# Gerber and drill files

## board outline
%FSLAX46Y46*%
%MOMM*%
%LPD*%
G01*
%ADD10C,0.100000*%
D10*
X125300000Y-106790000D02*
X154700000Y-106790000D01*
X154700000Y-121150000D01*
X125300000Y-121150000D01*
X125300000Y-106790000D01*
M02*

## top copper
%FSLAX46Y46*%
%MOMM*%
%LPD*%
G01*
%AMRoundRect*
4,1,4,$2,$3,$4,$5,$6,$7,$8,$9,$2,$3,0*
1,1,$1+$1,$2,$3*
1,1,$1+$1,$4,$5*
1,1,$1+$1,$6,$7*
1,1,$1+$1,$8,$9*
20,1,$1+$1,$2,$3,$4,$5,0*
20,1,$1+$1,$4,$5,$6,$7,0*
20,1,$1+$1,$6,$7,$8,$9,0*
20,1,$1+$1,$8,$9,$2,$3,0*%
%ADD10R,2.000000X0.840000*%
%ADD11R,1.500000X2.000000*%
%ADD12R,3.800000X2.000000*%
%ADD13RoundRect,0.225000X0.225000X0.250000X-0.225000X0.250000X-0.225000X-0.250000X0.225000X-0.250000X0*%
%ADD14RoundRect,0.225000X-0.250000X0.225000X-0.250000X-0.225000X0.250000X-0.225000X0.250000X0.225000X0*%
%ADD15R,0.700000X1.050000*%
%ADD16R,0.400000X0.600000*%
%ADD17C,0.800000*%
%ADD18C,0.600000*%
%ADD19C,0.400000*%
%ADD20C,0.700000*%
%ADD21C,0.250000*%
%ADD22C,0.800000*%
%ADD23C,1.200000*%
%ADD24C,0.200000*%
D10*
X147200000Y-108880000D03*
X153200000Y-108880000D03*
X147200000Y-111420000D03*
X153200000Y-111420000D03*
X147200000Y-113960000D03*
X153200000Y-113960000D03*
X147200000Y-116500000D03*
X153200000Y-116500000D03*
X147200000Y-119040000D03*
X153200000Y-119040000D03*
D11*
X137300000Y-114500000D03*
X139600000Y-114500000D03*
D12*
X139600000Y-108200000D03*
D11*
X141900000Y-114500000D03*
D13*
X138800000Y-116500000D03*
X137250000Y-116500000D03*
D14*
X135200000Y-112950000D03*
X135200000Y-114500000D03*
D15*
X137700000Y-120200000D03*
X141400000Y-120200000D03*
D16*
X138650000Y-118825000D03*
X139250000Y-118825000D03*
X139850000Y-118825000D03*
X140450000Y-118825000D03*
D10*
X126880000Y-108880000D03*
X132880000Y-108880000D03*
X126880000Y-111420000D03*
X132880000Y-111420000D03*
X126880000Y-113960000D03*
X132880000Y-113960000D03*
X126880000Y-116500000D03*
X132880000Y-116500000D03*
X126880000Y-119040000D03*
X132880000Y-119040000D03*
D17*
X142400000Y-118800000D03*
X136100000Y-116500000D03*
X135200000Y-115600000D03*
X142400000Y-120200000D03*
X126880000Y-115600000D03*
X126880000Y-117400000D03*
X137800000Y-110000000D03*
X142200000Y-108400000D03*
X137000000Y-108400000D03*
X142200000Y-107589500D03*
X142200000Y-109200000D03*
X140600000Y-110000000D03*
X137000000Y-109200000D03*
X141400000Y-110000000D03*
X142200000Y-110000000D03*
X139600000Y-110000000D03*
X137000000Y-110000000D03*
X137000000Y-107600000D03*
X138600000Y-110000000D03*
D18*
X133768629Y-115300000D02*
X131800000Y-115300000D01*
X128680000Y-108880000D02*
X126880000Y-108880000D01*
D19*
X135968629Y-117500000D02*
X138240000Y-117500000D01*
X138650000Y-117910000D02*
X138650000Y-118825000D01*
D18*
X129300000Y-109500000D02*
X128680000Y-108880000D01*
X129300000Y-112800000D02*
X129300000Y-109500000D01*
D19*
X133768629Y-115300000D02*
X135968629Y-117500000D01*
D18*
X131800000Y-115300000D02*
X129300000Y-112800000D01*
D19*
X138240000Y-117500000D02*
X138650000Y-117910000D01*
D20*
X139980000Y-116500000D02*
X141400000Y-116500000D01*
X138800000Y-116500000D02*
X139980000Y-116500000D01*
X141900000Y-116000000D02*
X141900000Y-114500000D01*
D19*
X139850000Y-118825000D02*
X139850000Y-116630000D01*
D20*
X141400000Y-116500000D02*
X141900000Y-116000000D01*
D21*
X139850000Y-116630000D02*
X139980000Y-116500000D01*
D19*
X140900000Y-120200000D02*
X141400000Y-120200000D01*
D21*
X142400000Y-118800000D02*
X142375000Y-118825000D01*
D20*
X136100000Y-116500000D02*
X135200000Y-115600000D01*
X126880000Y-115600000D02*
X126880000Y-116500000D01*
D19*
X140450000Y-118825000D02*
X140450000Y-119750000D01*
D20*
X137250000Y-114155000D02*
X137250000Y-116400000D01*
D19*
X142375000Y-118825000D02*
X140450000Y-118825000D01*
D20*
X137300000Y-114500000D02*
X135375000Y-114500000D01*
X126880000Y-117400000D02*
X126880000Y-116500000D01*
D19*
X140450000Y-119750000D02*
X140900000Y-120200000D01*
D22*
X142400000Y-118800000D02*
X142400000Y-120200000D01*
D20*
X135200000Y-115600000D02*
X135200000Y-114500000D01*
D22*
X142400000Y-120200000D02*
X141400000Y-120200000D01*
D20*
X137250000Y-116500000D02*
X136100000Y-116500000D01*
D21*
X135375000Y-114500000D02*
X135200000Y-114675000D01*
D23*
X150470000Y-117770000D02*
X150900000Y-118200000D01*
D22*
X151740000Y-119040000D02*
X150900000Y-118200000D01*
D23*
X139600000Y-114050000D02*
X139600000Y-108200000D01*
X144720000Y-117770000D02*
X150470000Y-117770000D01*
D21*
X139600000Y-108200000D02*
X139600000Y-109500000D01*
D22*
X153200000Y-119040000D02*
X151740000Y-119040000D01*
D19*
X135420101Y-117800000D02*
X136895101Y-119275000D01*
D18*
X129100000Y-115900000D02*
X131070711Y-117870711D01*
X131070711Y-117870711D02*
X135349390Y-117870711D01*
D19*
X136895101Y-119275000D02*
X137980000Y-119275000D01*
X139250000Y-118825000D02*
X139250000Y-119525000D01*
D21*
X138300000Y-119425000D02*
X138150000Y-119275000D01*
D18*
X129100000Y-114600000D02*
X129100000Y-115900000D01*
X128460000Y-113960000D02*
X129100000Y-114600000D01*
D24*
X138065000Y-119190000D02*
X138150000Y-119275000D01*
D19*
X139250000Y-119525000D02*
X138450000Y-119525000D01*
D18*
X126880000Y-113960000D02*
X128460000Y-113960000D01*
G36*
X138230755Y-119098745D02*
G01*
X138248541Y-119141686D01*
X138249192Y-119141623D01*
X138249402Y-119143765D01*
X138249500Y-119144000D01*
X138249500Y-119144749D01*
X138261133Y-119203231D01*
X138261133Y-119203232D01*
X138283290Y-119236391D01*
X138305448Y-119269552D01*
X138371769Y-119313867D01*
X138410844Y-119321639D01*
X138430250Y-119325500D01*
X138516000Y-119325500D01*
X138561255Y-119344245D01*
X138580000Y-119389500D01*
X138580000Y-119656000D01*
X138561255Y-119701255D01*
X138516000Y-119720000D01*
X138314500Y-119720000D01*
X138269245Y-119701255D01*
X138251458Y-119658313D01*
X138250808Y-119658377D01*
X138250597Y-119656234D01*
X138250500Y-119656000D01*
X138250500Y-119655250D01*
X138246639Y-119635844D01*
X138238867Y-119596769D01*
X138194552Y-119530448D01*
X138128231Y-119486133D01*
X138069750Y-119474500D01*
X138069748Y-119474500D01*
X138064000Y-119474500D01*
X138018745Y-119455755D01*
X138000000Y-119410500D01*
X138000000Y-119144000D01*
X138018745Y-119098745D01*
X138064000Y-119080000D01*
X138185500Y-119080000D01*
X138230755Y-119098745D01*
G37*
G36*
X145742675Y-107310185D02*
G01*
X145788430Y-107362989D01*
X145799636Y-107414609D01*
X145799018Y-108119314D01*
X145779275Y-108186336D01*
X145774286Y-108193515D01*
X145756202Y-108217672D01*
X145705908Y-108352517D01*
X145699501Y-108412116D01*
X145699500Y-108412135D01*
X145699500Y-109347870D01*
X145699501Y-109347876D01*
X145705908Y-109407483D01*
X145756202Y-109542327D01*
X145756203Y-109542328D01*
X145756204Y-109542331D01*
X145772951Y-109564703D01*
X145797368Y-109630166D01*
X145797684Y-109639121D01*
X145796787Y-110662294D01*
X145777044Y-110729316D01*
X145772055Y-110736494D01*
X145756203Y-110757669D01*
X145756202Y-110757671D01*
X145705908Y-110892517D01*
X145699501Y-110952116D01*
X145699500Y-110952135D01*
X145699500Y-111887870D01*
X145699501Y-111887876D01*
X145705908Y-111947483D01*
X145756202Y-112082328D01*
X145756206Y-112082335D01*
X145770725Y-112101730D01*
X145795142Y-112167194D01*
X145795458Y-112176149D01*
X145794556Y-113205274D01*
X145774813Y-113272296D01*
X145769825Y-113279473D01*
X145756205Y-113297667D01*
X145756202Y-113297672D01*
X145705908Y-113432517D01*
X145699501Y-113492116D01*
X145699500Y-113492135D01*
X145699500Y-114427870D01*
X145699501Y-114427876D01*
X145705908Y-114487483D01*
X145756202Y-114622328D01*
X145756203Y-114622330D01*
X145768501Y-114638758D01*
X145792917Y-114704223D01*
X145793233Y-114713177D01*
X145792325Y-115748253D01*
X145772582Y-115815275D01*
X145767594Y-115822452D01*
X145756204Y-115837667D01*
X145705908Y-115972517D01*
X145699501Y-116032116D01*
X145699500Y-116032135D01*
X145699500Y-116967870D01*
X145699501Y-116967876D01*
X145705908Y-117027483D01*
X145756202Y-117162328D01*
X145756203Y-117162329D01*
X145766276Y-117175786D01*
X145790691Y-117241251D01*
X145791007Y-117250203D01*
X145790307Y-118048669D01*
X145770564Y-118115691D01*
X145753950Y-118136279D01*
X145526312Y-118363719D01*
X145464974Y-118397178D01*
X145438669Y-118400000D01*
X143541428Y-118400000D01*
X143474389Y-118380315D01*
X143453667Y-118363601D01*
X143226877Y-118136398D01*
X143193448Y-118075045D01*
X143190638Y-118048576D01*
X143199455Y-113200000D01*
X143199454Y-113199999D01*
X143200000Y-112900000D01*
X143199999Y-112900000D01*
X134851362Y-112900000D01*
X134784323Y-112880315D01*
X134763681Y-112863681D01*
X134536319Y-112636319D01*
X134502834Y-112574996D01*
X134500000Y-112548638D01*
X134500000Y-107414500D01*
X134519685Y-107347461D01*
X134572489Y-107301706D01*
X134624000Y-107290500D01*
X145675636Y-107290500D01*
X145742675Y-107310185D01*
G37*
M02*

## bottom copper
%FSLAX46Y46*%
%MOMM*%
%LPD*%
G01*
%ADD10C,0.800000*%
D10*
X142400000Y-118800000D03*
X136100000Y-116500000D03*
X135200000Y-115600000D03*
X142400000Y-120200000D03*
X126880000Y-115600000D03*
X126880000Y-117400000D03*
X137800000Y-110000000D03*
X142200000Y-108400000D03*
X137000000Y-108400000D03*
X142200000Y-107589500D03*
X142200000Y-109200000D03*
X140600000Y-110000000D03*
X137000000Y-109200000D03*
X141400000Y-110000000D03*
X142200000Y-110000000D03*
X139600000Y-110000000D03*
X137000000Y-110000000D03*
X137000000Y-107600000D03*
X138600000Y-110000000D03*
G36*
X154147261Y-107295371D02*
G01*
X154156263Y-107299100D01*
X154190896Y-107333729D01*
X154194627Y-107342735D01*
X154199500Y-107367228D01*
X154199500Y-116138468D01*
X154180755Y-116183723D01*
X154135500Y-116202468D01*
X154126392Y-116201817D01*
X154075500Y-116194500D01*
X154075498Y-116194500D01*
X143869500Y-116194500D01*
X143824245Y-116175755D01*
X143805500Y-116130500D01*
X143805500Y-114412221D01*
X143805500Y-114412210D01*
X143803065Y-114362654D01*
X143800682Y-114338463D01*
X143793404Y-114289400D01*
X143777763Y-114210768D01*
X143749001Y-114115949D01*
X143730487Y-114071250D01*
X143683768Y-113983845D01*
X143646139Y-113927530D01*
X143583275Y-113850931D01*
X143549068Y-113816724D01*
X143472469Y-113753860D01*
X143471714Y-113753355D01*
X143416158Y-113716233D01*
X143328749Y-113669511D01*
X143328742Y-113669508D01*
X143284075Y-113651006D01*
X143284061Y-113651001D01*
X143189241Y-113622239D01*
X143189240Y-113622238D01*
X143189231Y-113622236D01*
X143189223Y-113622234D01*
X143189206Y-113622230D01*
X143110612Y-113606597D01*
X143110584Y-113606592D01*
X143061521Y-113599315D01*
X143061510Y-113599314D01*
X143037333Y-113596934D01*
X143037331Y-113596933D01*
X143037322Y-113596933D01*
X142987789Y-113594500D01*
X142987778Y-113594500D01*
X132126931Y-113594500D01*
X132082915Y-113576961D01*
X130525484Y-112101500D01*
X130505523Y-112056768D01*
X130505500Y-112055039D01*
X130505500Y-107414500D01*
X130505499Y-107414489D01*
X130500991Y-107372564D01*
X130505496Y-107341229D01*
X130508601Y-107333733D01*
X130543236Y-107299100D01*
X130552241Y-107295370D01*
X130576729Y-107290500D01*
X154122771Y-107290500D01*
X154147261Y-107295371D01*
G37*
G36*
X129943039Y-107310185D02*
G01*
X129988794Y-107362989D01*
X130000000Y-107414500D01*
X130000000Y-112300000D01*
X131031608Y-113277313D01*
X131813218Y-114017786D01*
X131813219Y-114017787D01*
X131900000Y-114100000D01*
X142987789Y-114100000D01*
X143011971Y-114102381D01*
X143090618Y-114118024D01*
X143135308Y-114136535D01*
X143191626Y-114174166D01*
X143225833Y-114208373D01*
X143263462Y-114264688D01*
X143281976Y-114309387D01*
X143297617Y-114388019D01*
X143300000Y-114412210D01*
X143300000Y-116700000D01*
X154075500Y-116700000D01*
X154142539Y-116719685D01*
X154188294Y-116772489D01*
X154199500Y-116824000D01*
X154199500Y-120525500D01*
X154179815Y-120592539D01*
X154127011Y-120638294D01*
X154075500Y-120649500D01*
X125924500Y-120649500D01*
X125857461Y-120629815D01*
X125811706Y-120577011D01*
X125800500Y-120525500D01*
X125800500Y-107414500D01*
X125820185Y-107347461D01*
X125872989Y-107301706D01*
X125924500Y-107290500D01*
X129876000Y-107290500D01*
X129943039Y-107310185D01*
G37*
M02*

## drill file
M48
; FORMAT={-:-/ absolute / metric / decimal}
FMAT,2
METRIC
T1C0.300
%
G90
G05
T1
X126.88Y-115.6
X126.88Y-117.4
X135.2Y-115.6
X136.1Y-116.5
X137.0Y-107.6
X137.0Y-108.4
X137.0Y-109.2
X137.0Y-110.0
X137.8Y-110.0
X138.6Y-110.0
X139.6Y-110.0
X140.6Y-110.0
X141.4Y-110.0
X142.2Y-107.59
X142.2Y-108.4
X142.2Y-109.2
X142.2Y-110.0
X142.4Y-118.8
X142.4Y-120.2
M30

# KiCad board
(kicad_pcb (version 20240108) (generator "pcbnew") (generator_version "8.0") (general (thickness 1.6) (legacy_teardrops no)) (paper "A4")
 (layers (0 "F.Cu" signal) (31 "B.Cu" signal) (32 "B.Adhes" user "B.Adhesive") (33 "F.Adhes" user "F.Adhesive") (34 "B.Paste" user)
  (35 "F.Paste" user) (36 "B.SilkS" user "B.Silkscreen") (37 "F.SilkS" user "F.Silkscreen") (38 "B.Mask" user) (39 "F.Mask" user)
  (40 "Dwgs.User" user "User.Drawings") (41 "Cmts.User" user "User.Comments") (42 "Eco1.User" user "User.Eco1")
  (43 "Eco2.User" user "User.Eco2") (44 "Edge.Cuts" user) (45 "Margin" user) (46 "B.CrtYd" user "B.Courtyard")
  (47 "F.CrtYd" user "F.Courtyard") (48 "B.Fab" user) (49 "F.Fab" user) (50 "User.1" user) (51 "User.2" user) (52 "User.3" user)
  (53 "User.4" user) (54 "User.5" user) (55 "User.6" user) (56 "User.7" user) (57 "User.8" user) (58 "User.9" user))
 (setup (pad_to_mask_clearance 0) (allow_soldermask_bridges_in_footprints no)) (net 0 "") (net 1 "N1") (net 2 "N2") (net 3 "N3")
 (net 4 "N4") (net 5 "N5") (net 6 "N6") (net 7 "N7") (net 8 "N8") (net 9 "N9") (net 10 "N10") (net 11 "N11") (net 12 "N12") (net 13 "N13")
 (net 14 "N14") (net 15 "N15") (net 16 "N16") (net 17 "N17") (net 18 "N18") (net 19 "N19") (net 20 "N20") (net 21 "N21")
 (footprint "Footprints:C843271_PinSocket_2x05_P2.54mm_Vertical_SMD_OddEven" (layer "F.Cu") (at 150.2 113.96)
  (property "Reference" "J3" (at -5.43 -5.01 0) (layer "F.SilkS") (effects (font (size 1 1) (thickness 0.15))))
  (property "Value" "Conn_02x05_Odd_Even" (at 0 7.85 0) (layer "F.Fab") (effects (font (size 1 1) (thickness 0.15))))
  (pad "1" smd rect (at -3 -5.08) (size 2 0.84) (layers "F.Cu" "F.Paste" "F.Mask") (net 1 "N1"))
  (pad "2" smd rect (at 3 -5.08) (size 2 0.84) (layers "F.Cu" "F.Paste" "F.Mask") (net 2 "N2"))
  (pad "3" smd rect (at -3 -2.54) (size 2 0.84) (layers "F.Cu" "F.Paste" "F.Mask") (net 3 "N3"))
  (pad "4" smd rect (at 3 -2.54) (size 2 0.84) (layers "F.Cu" "F.Paste" "F.Mask") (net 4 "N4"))
  (pad "5" smd rect (at -3 0) (size 2 0.84) (layers "F.Cu" "F.Paste" "F.Mask") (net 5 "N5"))
  (pad "6" smd rect (at 3 0) (size 2 0.84) (layers "F.Cu" "F.Paste" "F.Mask") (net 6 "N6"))
  (pad "7" smd rect (at -3 2.54) (size 2 0.84) (layers "F.Cu" "F.Paste" "F.Mask") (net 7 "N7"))
  (pad "8" smd rect (at 3 2.54) (size 2 0.84) (layers "F.Cu" "F.Paste" "F.Mask") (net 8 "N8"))
  (pad "9" smd rect (at -3 5.08) (size 2 0.84) (layers "F.Cu" "F.Paste" "F.Mask") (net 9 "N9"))
  (pad "10" smd rect (at 3 5.08) (size 2 0.84) (layers "F.Cu" "F.Paste" "F.Mask") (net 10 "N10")))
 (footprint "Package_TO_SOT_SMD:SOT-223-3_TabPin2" (layer "F.Cu") (at 139.6 111.35 90)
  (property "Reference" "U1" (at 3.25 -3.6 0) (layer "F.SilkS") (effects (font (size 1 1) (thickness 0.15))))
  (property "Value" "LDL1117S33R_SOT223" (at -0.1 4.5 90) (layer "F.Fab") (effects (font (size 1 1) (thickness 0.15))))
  (pad "1" smd rect (at -3.15 -2.3 90) (size 2 1.5) (layers "F.Cu" "F.Paste" "F.Mask") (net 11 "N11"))
  (pad "2" smd rect (at -3.15 0 90) (size 2 1.5) (layers "F.Cu" "F.Paste" "F.Mask") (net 10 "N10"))
  (pad "2" smd rect (at 3.15 0 90) (size 2 3.8) (layers "F.Cu" "F.Paste" "F.Mask") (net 10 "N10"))
  (pad "3" smd rect (at -3.15 2.3 90) (size 2 1.5) (layers "F.Cu" "F.Paste" "F.Mask") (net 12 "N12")))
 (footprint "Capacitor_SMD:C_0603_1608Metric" (layer "F.Cu") (at 138.025 116.5 180)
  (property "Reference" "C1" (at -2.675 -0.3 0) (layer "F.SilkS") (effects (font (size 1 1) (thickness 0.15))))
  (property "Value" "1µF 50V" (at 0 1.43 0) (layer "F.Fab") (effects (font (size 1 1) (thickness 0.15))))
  (pad "1" smd roundrect (at -0.775 0 180) (size 0.9 0.95) (layers "F.Cu" "F.Paste" "F.Mask") (roundrect_rratio 0.25) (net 12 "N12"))
  (pad "2" smd roundrect (at 0.775 0 180) (size 0.9 0.95) (layers "F.Cu" "F.Paste" "F.Mask") (roundrect_rratio 0.25) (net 11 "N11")))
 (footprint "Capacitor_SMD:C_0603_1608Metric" (layer "F.Cu") (at 135.2 113.725 -90)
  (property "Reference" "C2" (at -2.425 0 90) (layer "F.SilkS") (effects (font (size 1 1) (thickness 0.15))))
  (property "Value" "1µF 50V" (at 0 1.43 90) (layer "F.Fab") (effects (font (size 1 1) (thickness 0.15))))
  (pad "1" smd roundrect (at -0.775 0 270) (size 0.9 0.95) (layers "F.Cu" "F.Paste" "F.Mask") (roundrect_rratio 0.25) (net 10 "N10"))
  (pad "2" smd roundrect (at 0.775 0 270) (size 0.9 0.95) (layers "F.Cu" "F.Paste" "F.Mask") (roundrect_rratio 0.25) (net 11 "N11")))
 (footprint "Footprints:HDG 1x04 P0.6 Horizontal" (layer "F.Cu") (at 139.55 120.575)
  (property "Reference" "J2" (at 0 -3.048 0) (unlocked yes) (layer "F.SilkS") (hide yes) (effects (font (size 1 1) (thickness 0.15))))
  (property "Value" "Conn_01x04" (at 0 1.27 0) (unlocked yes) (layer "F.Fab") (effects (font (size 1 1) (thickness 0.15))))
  (pad "" smd rect (at -1.85 -0.375 90) (size 1.05 0.7) (layers "F.Cu" "F.Paste" "F.Mask") (thermal_bridge_angle 45))
  (pad "" smd rect (at 1.85 -0.375 90) (size 1.05 0.7) (layers "F.Cu" "F.Paste" "F.Mask") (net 11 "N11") (thermal_bridge_angle 45))
  (pad "1" smd rect (at -0.9 -1.75 90) (size 0.6 0.4) (layers "F.Cu" "F.Paste" "F.Mask") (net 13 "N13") (thermal_bridge_angle 45))
  (pad "2" smd rect (at -0.3 -1.75 90) (size 0.6 0.4) (layers "F.Cu" "F.Paste" "F.Mask") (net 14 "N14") (thermal_bridge_angle 45))
  (pad "3" smd rect (at 0.3 -1.75 90) (size 0.6 0.4) (layers "F.Cu" "F.Paste" "F.Mask") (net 12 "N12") (thermal_bridge_angle 45))
  (pad "4" smd rect (at 0.9 -1.75 90) (size 0.6 0.4) (layers "F.Cu" "F.Paste" "F.Mask") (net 11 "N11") (thermal_bridge_angle 45)))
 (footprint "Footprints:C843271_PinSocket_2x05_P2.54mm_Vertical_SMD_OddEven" (layer "F.Cu") (at 129.88 113.96)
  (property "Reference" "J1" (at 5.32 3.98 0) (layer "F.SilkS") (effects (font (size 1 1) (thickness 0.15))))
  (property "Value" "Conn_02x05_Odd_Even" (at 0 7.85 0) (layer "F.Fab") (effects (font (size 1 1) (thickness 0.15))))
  (pad "1" smd rect (at -3 -5.08) (size 2 0.84) (layers "F.Cu" "F.Paste" "F.Mask") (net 13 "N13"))
  (pad "2" smd rect (at 3 -5.08) (size 2 0.84) (layers "F.Cu" "F.Paste" "F.Mask") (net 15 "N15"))
  (pad "3" smd rect (at -3 -2.54) (size 2 0.84) (layers "F.Cu" "F.Paste" "F.Mask") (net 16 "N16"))
  (pad "4" smd rect (at 3 -2.54) (size 2 0.84) (layers "F.Cu" "F.Paste" "F.Mask") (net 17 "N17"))
  (pad "5" smd rect (at -3 0) (size 2 0.84) (layers "F.Cu" "F.Paste" "F.Mask") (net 14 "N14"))
  (pad "6" smd rect (at 3 0) (size 2 0.84) (layers "F.Cu" "F.Paste" "F.Mask") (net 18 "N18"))
  (pad "7" smd rect (at -3 2.54) (size 2 0.84) (layers "F.Cu" "F.Paste" "F.Mask") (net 11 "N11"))
  (pad "8" smd rect (at 3 2.54) (size 2 0.84) (layers "F.Cu" "F.Paste" "F.Mask") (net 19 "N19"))
  (pad "9" smd rect (at -3 5.08) (size 2 0.84) (layers "F.Cu" "F.Paste" "F.Mask") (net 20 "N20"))
  (pad "10" smd rect (at 3 5.08) (size 2 0.84) (layers "F.Cu" "F.Paste" "F.Mask") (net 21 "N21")))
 (gr_rect (start 125.3 106.79) (end 154.7 121.15) (stroke (width 0.1) (type default)) (fill none) (layer "Edge.Cuts"))
 (segment (start 133.768629 115.3) (end 131.8 115.3) (width 0.6) (layer "F.Cu") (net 13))
 (segment (start 128.68 108.88) (end 126.88 108.88) (width 0.6) (layer "F.Cu") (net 13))
 (segment (start 135.968629 117.5) (end 138.24 117.5) (width 0.4) (layer "F.Cu") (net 13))
 (segment (start 138.65 117.91) (end 138.65 118.825) (width 0.4) (layer "F.Cu") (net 13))
 (segment (start 129.3 109.5) (end 128.68 108.88) (width 0.6) (layer "F.Cu") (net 13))
 (segment (start 129.3 112.8) (end 129.3 109.5) (width 0.6) (layer "F.Cu") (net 13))
 (segment (start 133.768629 115.3) (end 135.968629 117.5) (width 0.4) (layer "F.Cu") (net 13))
 (segment (start 131.8 115.3) (end 129.3 112.8) (width 0.6) (layer "F.Cu") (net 13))
 (segment (start 138.24 117.5) (end 138.65 117.91) (width 0.4) (layer "F.Cu") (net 13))
 (segment (start 139.98 116.5) (end 141.4 116.5) (width 0.7) (layer "F.Cu") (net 12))
 (segment (start 138.8 116.5) (end 139.98 116.5) (width 0.7) (layer "F.Cu") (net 12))
 (segment (start 141.9 116) (end 141.9 114.5) (width 0.7) (layer "F.Cu") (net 12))
 (segment (start 139.85 118.825) (end 139.85 116.63) (width 0.4) (layer "F.Cu") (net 12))
 (segment (start 141.4 116.5) (end 141.9 116) (width 0.7) (layer "F.Cu") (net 12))
 (segment (start 139.85 116.63) (end 139.98 116.5) (width 0.25) (layer "F.Cu") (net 12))
 (segment (start 140.9 120.2) (end 141.4 120.2) (width 0.4) (layer "F.Cu") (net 11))
 (segment (start 142.4 118.8) (end 142.375 118.825) (width 0.25) (layer "F.Cu") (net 11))
 (segment (start 136.1 116.5) (end 135.2 115.6) (width 0.7) (layer "F.Cu") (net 11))
 (segment (start 126.88 115.6) (end 126.88 116.5) (width 0.7) (layer "F.Cu") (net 11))
 (segment (start 140.45 118.825) (end 140.45 119.75) (width 0.4) (layer "F.Cu") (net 11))
 (segment (start 137.25 114.155) (end 137.25 116.4) (width 0.7) (layer "F.Cu") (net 11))
 (segment (start 142.375 118.825) (end 140.45 118.825) (width 0.4) (layer "F.Cu") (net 11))
 (segment (start 137.3 114.5) (end 135.375 114.5) (width 0.7) (layer "F.Cu") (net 11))
 (segment (start 126.88 117.4) (end 126.88 116.5) (width 0.7) (layer "F.Cu") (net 11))
 (segment (start 140.45 119.75) (end 140.9 120.2) (width 0.4) (layer "F.Cu") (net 11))
 (segment (start 142.4 118.8) (end 142.4 120.2) (width 0.8) (layer "F.Cu") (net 11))
 (segment (start 135.2 115.6) (end 135.2 114.5) (width 0.7) (layer "F.Cu") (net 11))
 (segment (start 142.4 120.2) (end 141.4 120.2) (width 0.8) (layer "F.Cu") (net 11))
 (segment (start 137.25 116.5) (end 136.1 116.5) (width 0.7) (layer "F.Cu") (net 11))
 (segment (start 135.375 114.5) (end 135.2 114.675) (width 0.25) (layer "F.Cu") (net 11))
 (via (at 142.4 118.8) (size 0.8) (drill 0.3) (layers "F.Cu" "B.Cu") (free yes) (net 11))
 (via (at 136.1 116.5) (size 0.8) (drill 0.3) (layers "F.Cu" "B.Cu") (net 11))
 (via (at 135.2 115.6) (size 0.8) (drill 0.3) (layers "F.Cu" "B.Cu") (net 11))
 (via (at 142.4 120.2) (size 0.8) (drill 0.3) (layers "F.Cu" "B.Cu") (free yes) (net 11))
 (via (at 126.88 115.6) (size 0.8) (drill 0.3) (layers "F.Cu" "B.Cu") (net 11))
 (via (at 126.88 117.4) (size 0.8) (drill 0.3) (layers "F.Cu" "B.Cu") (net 11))
 (segment (start 150.47 117.77) (end 150.9 118.2) (width 1.2) (layer "F.Cu") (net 10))
 (segment (start 151.74 119.04) (end 150.9 118.2) (width 0.8) (layer "F.Cu") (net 10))
 (segment (start 139.6 114.05) (end 139.6 108.2) (width 1.2) (layer "F.Cu") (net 10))
 (segment (start 144.72 117.77) (end 150.47 117.77) (width 1.2) (layer "F.Cu") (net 10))
 (segment (start 139.6 108.2) (end 139.6 109.5) (width 0.25) (layer "F.Cu") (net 10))
 (segment (start 153.2 119.04) (end 151.74 119.04) (width 0.8) (layer "F.Cu") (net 10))
 (via (at 137.8 110) (size 0.8) (drill 0.3) (layers "F.Cu" "B.Cu") (free yes) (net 10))
 (via (at 142.2 108.4) (size 0.8) (drill 0.3) (layers "F.Cu" "B.Cu") (free yes) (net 10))
 (via (at 137 108.4) (size 0.8) (drill 0.3) (layers "F.Cu" "B.Cu") (free yes) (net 10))
 (via (at 142.2 107.5895) (size 0.8) (drill 0.3) (layers "F.Cu" "B.Cu") (free yes) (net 10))
 (via (at 142.2 109.2) (size 0.8) (drill 0.3) (layers "F.Cu" "B.Cu") (free yes) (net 10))
 (via (at 140.6 110) (size 0.8) (drill 0.3) (layers "F.Cu" "B.Cu") (free yes) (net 10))
 (via (at 137 109.2) (size 0.8) (drill 0.3) (layers "F.Cu" "B.Cu") (free yes) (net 10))
 (via (at 141.4 110) (size 0.8) (drill 0.3) (layers "F.Cu" "B.Cu") (free yes) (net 10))
 (via (at 142.2 110) (size 0.8) (drill 0.3) (layers "F.Cu" "B.Cu") (free yes) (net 10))
 (via (at 139.6 110) (size 0.8) (drill 0.3) (layers "F.Cu" "B.Cu") (free yes) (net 10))
 (via (at 137 110) (size 0.8) (drill 0.3) (layers "F.Cu" "B.Cu") (free yes) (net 10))
 (via (at 137 107.6) (size 0.8) (drill 0.3) (layers "F.Cu" "B.Cu") (free yes) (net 10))
 (via (at 138.6 110) (size 0.8) (drill 0.3) (layers "F.Cu" "B.Cu") (free yes) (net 10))
 (segment (start 135.420101 117.8) (end 136.895101 119.275) (width 0.4) (layer "F.Cu") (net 14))
 (segment (start 129.1 115.9) (end 131.070711 117.870711) (width 0.6) (layer "F.Cu") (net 14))
 (segment (start 131.070711 117.870711) (end 135.34939 117.870711) (width 0.6) (layer "F.Cu") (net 14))
 (segment (start 136.895101 119.275) (end 137.98 119.275) (width 0.4) (layer "F.Cu") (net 14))
 (segment (start 139.25 118.825) (end 139.25 119.525) (width 0.4) (layer "F.Cu") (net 14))
 (segment (start 138.3 119.425) (end 138.15 119.275) (width 0.25) (layer "F.Cu") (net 14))
 (segment (start 129.1 114.6) (end 129.1 115.9) (width 0.6) (layer "F.Cu") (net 14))
 (segment (start 128.46 113.96) (end 129.1 114.6) (width 0.6) (layer "F.Cu") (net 14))
 (segment (start 138.065 119.19) (end 138.15 119.275) (width 0.2) (layer "F.Cu") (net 14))
 (segment (start 139.25 119.525) (end 138.45 119.525) (width 0.4) (layer "F.Cu") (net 14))
 (segment (start 126.88 113.96) (end 128.46 113.96) (width 0.6) (layer "F.Cu") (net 14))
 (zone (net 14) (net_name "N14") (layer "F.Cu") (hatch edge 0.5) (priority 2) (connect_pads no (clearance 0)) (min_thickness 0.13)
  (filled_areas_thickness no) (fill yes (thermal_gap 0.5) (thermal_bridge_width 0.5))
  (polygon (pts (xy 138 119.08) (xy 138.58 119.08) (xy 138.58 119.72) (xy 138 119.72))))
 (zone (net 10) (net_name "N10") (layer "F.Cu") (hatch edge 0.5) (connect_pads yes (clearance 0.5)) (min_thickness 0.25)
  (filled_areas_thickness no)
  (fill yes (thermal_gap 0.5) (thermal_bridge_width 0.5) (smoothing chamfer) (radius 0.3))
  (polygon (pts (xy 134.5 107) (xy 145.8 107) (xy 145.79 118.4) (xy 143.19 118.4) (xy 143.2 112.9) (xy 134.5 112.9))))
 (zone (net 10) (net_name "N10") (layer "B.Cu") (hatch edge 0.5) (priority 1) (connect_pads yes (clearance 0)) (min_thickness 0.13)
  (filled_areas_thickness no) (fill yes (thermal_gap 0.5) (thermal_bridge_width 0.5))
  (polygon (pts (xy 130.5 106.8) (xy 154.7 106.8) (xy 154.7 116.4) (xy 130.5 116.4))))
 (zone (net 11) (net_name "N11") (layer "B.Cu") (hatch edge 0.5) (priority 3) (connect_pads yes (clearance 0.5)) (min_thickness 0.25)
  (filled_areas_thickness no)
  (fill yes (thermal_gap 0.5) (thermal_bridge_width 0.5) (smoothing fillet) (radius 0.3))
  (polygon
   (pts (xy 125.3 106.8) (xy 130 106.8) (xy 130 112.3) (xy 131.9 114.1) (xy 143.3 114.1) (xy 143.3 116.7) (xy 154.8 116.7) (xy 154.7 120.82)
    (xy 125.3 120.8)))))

